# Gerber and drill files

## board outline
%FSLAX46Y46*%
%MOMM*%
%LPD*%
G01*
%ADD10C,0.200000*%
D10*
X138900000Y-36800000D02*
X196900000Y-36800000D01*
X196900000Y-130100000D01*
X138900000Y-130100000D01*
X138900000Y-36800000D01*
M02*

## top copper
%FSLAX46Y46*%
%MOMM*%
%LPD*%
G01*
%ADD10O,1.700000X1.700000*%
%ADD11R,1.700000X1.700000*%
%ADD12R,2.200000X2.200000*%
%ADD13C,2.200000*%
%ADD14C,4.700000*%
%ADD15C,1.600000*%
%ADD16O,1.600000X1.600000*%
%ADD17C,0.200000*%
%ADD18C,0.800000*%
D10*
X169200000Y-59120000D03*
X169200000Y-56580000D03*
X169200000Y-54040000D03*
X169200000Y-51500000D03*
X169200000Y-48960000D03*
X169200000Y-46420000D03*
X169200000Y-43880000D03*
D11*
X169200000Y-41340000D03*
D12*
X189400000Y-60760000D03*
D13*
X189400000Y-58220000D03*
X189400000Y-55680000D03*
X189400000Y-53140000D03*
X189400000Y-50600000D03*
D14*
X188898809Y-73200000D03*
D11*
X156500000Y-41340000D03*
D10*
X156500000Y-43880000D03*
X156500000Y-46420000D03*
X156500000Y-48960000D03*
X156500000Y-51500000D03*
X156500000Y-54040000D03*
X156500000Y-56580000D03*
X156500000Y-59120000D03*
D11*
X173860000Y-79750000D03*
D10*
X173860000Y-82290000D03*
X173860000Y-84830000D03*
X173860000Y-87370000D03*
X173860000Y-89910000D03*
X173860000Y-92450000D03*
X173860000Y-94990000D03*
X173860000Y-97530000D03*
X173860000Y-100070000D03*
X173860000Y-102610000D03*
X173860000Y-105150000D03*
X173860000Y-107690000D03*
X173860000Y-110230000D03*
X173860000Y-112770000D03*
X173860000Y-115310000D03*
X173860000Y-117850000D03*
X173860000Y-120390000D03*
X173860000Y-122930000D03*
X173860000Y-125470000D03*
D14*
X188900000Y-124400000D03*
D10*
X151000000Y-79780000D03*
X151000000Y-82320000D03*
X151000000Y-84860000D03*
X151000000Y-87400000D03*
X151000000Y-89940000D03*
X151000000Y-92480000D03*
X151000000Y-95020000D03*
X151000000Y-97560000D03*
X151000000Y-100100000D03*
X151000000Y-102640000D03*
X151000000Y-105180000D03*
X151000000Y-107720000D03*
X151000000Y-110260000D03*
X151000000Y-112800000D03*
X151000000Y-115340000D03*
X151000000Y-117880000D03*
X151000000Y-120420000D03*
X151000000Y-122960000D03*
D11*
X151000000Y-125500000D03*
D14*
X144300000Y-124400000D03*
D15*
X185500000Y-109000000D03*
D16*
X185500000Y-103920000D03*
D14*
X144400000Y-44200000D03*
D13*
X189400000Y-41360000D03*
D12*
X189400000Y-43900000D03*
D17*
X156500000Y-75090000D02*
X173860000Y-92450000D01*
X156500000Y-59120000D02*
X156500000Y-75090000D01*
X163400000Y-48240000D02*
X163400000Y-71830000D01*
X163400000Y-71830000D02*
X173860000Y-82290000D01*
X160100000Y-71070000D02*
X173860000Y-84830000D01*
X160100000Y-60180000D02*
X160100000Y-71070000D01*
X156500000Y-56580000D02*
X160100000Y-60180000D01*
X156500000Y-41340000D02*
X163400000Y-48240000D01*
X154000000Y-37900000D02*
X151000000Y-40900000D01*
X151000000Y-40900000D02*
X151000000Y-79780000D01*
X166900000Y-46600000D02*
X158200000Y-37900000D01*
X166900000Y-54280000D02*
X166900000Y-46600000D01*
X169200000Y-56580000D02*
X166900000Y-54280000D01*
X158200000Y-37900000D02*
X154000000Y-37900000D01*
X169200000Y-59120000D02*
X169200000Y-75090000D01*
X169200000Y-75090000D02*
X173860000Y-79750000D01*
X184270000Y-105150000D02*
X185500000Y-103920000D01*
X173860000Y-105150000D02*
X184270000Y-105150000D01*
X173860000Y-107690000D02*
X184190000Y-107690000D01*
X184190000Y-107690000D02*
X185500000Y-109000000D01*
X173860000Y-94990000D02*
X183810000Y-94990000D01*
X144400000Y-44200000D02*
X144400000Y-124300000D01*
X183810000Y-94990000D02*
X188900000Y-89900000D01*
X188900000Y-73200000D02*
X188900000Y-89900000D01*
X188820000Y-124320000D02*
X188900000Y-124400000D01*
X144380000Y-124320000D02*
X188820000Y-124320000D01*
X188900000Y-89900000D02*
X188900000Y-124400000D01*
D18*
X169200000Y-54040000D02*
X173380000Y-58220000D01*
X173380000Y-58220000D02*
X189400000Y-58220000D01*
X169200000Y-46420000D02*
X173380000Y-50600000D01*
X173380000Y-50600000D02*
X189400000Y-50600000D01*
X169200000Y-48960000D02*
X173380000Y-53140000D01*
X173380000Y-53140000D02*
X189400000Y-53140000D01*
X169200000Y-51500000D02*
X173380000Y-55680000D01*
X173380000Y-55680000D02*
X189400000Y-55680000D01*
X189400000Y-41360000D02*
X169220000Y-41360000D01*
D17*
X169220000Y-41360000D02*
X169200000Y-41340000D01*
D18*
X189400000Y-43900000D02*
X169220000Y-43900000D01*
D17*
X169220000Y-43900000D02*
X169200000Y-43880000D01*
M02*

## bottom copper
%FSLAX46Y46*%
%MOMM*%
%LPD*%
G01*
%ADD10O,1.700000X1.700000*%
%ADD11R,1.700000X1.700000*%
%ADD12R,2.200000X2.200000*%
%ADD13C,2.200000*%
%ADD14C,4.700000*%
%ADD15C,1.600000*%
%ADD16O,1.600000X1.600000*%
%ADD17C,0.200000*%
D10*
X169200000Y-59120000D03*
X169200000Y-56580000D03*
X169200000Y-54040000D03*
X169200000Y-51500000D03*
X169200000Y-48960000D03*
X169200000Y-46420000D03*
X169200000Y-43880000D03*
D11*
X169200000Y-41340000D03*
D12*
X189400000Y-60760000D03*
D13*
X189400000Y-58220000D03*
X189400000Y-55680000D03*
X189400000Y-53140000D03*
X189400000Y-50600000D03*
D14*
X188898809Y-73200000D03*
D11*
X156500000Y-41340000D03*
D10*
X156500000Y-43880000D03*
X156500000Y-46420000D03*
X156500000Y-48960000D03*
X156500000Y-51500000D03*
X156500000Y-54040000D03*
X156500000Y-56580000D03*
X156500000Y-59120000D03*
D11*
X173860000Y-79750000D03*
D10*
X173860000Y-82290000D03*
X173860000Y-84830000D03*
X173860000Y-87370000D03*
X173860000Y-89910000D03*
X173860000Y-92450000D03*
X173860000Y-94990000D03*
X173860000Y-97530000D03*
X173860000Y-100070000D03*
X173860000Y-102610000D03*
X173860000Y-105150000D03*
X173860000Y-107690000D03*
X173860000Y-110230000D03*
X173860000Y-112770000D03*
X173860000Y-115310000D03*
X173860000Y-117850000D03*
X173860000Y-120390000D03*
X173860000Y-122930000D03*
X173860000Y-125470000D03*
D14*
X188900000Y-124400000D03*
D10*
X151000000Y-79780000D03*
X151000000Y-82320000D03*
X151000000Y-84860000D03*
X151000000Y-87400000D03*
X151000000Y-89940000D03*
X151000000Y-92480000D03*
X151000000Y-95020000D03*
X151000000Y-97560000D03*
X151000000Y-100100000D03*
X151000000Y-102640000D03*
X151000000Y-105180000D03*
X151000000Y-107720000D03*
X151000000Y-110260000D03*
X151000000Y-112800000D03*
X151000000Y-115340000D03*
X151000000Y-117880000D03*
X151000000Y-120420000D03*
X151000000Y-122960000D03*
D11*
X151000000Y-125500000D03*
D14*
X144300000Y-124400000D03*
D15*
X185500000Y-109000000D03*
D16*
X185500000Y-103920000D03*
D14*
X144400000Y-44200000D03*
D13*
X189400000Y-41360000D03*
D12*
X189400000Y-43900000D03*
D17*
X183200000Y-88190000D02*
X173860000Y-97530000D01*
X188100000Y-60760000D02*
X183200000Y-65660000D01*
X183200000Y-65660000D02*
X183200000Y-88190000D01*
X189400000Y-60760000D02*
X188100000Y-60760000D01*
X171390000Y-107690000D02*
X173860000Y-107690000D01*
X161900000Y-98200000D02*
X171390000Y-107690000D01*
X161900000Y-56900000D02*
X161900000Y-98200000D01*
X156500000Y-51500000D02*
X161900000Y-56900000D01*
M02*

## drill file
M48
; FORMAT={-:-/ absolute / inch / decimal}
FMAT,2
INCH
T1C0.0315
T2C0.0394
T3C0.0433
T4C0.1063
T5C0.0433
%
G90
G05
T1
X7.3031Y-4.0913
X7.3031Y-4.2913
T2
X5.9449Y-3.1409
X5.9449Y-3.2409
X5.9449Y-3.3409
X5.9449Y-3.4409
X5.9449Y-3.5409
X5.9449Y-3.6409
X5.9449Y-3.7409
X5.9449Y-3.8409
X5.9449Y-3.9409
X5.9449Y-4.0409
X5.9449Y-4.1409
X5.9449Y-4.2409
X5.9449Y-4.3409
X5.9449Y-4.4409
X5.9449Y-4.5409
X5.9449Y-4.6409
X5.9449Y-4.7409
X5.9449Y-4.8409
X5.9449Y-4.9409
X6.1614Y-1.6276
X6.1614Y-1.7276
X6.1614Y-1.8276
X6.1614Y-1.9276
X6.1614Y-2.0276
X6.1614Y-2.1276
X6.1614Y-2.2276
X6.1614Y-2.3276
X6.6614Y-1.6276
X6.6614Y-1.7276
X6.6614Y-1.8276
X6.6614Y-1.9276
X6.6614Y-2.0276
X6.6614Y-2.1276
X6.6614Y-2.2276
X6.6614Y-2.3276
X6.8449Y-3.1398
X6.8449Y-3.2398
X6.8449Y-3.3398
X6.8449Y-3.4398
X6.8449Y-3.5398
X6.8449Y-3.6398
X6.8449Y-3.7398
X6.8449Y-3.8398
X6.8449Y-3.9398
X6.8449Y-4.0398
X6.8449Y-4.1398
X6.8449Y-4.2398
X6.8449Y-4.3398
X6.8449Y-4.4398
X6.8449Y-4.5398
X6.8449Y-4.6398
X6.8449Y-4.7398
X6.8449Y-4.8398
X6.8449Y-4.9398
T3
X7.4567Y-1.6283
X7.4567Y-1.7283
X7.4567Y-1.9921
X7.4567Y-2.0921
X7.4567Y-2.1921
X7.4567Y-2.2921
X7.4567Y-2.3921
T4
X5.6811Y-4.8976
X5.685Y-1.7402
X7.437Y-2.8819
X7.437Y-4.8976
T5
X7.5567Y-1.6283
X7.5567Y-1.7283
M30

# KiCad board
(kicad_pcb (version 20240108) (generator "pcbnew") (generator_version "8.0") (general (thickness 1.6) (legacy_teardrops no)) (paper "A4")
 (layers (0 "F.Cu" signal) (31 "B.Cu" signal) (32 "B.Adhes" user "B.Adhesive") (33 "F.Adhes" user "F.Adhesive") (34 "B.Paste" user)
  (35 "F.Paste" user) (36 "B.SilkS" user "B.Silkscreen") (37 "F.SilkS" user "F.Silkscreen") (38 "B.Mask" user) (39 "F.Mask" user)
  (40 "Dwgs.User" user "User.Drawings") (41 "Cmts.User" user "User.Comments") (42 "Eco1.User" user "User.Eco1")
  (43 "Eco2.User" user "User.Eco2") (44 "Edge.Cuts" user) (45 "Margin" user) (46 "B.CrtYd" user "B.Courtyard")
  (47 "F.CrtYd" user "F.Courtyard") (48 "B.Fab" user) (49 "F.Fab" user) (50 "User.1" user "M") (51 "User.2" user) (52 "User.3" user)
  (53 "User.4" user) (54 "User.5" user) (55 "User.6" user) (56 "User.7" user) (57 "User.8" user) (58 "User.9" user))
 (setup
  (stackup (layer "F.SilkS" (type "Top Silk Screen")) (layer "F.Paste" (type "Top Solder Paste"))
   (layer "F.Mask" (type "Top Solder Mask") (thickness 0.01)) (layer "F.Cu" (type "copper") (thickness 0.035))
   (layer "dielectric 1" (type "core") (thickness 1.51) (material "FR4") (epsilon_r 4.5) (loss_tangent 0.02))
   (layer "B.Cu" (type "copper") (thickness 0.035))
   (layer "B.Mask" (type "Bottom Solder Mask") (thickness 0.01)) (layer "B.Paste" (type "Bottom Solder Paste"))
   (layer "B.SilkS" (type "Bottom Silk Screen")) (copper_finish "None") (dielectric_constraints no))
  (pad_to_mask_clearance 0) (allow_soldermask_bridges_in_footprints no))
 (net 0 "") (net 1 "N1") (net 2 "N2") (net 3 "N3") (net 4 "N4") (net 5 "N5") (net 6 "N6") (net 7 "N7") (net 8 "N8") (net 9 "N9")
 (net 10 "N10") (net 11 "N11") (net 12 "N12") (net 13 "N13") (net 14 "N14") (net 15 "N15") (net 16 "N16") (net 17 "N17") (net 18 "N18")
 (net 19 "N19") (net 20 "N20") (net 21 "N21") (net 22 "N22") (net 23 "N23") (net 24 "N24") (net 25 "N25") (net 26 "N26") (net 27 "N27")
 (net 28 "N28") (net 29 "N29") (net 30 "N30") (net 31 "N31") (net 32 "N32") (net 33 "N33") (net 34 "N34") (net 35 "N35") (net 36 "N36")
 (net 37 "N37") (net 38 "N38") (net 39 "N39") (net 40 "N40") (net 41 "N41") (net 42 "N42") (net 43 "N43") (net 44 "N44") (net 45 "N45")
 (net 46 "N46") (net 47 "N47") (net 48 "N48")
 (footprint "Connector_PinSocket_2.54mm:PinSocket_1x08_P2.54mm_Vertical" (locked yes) (layer "F.Cu") (at 169.2 41.34)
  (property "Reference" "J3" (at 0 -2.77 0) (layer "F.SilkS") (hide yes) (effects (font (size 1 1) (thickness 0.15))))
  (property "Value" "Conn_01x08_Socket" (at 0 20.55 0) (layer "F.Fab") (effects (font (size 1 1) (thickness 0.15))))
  (pad "1" thru_hole rect (at 0 0) (size 1.7 1.7) (drill 1) (layers "*.Cu" "*.Mask") (remove_unused_layers no) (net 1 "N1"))
  (pad "2" thru_hole oval (at 0 2.54) (size 1.7 1.7) (drill 1) (layers "*.Cu" "*.Mask") (remove_unused_layers no) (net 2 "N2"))
  (pad "3" thru_hole oval (at 0 5.08) (size 1.7 1.7) (drill 1) (layers "*.Cu" "*.Mask") (remove_unused_layers no) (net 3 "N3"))
  (pad "4" thru_hole oval (at 0 7.62) (size 1.7 1.7) (drill 1) (layers "*.Cu" "*.Mask") (remove_unused_layers no) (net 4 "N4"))
  (pad "5" thru_hole oval (at 0 10.16) (size 1.7 1.7) (drill 1) (layers "*.Cu" "*.Mask") (remove_unused_layers no) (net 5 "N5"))
  (pad "6" thru_hole oval (at 0 12.7) (size 1.7 1.7) (drill 1) (layers "*.Cu" "*.Mask") (remove_unused_layers no) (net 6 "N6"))
  (pad "7" thru_hole oval (at 0 15.24) (size 1.7 1.7) (drill 1) (layers "*.Cu" "*.Mask") (remove_unused_layers no) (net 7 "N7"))
  (pad "8" thru_hole oval (at 0 17.78) (size 1.7 1.7) (drill 1) (layers "*.Cu" "*.Mask") (remove_unused_layers no) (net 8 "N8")))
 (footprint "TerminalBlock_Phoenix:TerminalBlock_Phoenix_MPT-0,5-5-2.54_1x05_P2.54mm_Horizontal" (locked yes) (layer "F.Cu")
  (at 189.4 60.76 90)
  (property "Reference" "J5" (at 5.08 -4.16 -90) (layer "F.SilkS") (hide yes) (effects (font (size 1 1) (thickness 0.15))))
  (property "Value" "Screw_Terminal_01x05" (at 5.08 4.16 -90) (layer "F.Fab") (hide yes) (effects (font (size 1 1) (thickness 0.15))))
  (pad "1" thru_hole rect (at 0 0 90) (size 2.2 2.2) (drill 1.1) (layers "*.Cu" "*.Mask") (remove_unused_layers no) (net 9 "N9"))
  (pad "2" thru_hole circle (at 2.54 0 90) (size 2.2 2.2) (drill 1.1) (layers "*.Cu" "*.Mask") (remove_unused_layers no) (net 6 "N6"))
  (pad "3" thru_hole circle (at 5.08 0 90) (size 2.2 2.2) (drill 1.1) (layers "*.Cu" "*.Mask") (remove_unused_layers no) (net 5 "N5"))
  (pad "4" thru_hole circle (at 7.62 0 90) (size 2.2 2.2) (drill 1.1) (layers "*.Cu" "*.Mask") (remove_unused_layers no) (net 4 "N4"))
  (pad "5" thru_hole circle (at 10.16 0 90) (size 2.2 2.2) (drill 1.1) (layers "*.Cu" "*.Mask") (remove_unused_layers no) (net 3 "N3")))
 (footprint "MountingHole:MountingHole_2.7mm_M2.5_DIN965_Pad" (layer "F.Cu") (at 188.898809 73.2)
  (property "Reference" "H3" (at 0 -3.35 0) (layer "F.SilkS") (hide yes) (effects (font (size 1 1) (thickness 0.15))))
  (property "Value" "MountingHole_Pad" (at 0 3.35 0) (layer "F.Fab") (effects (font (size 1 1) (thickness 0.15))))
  (pad "1" thru_hole circle (at 0 0) (size 4.7 4.7) (drill 2.7) (layers "*.Cu" "*.Mask") (remove_unused_layers no) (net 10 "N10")))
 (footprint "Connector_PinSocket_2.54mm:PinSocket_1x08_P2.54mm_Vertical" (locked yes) (layer "F.Cu") (at 156.5 41.34)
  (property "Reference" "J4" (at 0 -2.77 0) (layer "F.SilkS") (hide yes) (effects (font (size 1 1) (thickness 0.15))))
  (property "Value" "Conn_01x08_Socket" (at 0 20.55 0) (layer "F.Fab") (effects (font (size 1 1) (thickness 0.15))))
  (pad "1" thru_hole rect (at 0 0) (size 1.7 1.7) (drill 1) (layers "*.Cu" "*.Mask") (remove_unused_layers no) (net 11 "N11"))
  (pad "2" thru_hole oval (at 0 2.54) (size 1.7 1.7) (drill 1) (layers "*.Cu" "*.Mask") (remove_unused_layers no) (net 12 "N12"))
  (pad "3" thru_hole oval (at 0 5.08) (size 1.7 1.7) (drill 1) (layers "*.Cu" "*.Mask") (remove_unused_layers no) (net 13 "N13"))
  (pad "4" thru_hole oval (at 0 7.62) (size 1.7 1.7) (drill 1) (layers "*.Cu" "*.Mask") (remove_unused_layers no) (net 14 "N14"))
  (pad "5" thru_hole oval (at 0 10.16) (size 1.7 1.7) (drill 1) (layers "*.Cu" "*.Mask") (remove_unused_layers no) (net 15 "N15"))
  (pad "6" thru_hole oval (at 0 12.7) (size 1.7 1.7) (drill 1) (layers "*.Cu" "*.Mask") (remove_unused_layers no) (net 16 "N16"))
  (pad "7" thru_hole oval (at 0 15.24) (size 1.7 1.7) (drill 1) (layers "*.Cu" "*.Mask") (remove_unused_layers no) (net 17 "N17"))
  (pad "8" thru_hole oval (at 0 17.78) (size 1.7 1.7) (drill 1) (layers "*.Cu" "*.Mask") (remove_unused_layers no) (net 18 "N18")))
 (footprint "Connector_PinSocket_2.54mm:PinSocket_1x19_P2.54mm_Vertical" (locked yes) (layer "F.Cu") (at 173.86 79.75)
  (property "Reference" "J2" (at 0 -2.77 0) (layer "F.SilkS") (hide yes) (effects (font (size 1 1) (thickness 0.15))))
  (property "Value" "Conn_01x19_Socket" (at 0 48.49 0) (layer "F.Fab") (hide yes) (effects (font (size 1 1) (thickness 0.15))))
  (pad "1" thru_hole rect (at 0 0) (size 1.7 1.7) (drill 1) (layers "*.Cu" "*.Mask") (remove_unused_layers no) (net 8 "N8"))
  (pad "2" thru_hole oval (at 0 2.54) (size 1.7 1.7) (drill 1) (layers "*.Cu" "*.Mask") (remove_unused_layers no) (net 11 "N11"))
  (pad "3" thru_hole oval (at 0 5.08) (size 1.7 1.7) (drill 1) (layers "*.Cu" "*.Mask") (remove_unused_layers no) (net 17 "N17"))
  (pad "4" thru_hole oval (at 0 7.62) (size 1.7 1.7) (drill 1) (layers "*.Cu" "*.Mask") (remove_unused_layers no) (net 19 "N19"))
  (pad "5" thru_hole oval (at 0 10.16) (size 1.7 1.7) (drill 1) (layers "*.Cu" "*.Mask") (remove_unused_layers no) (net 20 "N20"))
  (pad "6" thru_hole oval (at 0 12.7) (size 1.7 1.7) (drill 1) (layers "*.Cu" "*.Mask") (remove_unused_layers no) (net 18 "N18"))
  (pad "7" thru_hole oval (at 0 15.24) (size 1.7 1.7) (drill 1) (layers "*.Cu" "*.Mask") (remove_unused_layers no) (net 10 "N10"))
  (pad "8" thru_hole oval (at 0 17.78) (size 1.7 1.7) (drill 1) (layers "*.Cu" "*.Mask") (remove_unused_layers no) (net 9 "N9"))
  (pad "9" thru_hole oval (at 0 20.32) (size 1.7 1.7) (drill 1) (layers "*.Cu" "*.Mask") (remove_unused_layers no) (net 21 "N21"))
  (pad "10" thru_hole oval (at 0 22.86) (size 1.7 1.7) (drill 1) (layers "*.Cu" "*.Mask") (remove_unused_layers no) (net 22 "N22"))
  (pad "11" thru_hole oval (at 0 25.4) (size 1.7 1.7) (drill 1) (layers "*.Cu" "*.Mask") (remove_unused_layers no) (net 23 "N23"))
  (pad "12" thru_hole oval (at 0 27.94) (size 1.7 1.7) (drill 1) (layers "*.Cu" "*.Mask") (remove_unused_layers no) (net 15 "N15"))
  (pad "13" thru_hole oval (at 0 30.48) (size 1.7 1.7) (drill 1) (layers "*.Cu" "*.Mask") (remove_unused_layers no) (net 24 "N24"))
  (pad "14" thru_hole oval (at 0 33.02) (size 1.7 1.7) (drill 1) (layers "*.Cu" "*.Mask") (remove_unused_layers no) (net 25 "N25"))
  (pad "15" thru_hole oval (at 0 35.56) (size 1.7 1.7) (drill 1) (layers "*.Cu" "*.Mask") (remove_unused_layers no) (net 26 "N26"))
  (pad "16" thru_hole oval (at 0 38.1) (size 1.7 1.7) (drill 1) (layers "*.Cu" "*.Mask") (remove_unused_layers no) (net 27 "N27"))
  (pad "17" thru_hole oval (at 0 40.64) (size 1.7 1.7) (drill 1) (layers "*.Cu" "*.Mask") (remove_unused_layers no) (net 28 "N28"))
  (pad "18" thru_hole oval (at 0 43.18) (size 1.7 1.7) (drill 1) (layers "*.Cu" "*.Mask") (remove_unused_layers no) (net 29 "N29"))
  (pad "19" thru_hole oval (at 0 45.72) (size 1.7 1.7) (drill 1) (layers "*.Cu" "*.Mask") (remove_unused_layers no) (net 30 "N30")))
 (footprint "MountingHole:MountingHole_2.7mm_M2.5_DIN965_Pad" (layer "F.Cu") (at 188.9 124.4)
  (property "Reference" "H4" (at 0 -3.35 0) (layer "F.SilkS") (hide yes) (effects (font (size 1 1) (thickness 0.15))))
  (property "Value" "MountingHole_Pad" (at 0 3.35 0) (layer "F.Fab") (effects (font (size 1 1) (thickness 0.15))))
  (pad "1" thru_hole circle (at 0 0) (size 4.7 4.7) (drill 2.7) (layers "*.Cu" "*.Mask") (remove_unused_layers no) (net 10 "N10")))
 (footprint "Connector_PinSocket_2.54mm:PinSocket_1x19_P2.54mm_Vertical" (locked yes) (layer "F.Cu") (at 151 125.5 180)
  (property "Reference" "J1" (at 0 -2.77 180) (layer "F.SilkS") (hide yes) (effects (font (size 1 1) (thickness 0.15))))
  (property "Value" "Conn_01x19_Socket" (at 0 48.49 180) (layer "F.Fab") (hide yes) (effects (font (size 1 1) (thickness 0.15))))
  (pad "1" thru_hole rect (at 0 0 180) (size 1.7 1.7) (drill 1) (layers "*.Cu" "*.Mask") (remove_unused_layers no) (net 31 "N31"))
  (pad "2" thru_hole oval (at 0 2.54 180) (size 1.7 1.7) (drill 1) (layers "*.Cu" "*.Mask") (remove_unused_layers no) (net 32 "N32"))
  (pad "3" thru_hole oval (at 0 5.08 180) (size 1.7 1.7) (drill 1) (layers "*.Cu" "*.Mask") (remove_unused_layers no) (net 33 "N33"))
  (pad "4" thru_hole oval (at 0 7.62 180) (size 1.7 1.7) (drill 1) (layers "*.Cu" "*.Mask") (remove_unused_layers no) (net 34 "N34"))
  (pad "5" thru_hole oval (at 0 10.16 180) (size 1.7 1.7) (drill 1) (layers "*.Cu" "*.Mask") (remove_unused_layers no) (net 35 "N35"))
  (pad "6" thru_hole oval (at 0 12.7 180) (size 1.7 1.7) (drill 1) (layers "*.Cu" "*.Mask") (remove_unused_layers no) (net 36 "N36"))
  (pad "7" thru_hole oval (at 0 15.24 180) (size 1.7 1.7) (drill 1) (layers "*.Cu" "*.Mask") (remove_unused_layers no) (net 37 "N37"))
  (pad "8" thru_hole oval (at 0 17.78 180) (size 1.7 1.7) (drill 1) (layers "*.Cu" "*.Mask") (remove_unused_layers no) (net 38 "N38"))
  (pad "9" thru_hole oval (at 0 20.32 180) (size 1.7 1.7) (drill 1) (layers "*.Cu" "*.Mask") (remove_unused_layers no) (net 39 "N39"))
  (pad "10" thru_hole oval (at 0 22.86 180) (size 1.7 1.7) (drill 1) (layers "*.Cu" "*.Mask") (remove_unused_layers no) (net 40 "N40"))
  (pad "11" thru_hole oval (at 0 25.4 180) (size 1.7 1.7) (drill 1) (layers "*.Cu" "*.Mask") (remove_unused_layers no) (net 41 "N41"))
  (pad "12" thru_hole oval (at 0 27.94 180) (size 1.7 1.7) (drill 1) (layers "*.Cu" "*.Mask") (remove_unused_layers no) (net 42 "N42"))
  (pad "13" thru_hole oval (at 0 30.48 180) (size 1.7 1.7) (drill 1) (layers "*.Cu" "*.Mask") (remove_unused_layers no) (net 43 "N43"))
  (pad "14" thru_hole oval (at 0 33.02 180) (size 1.7 1.7) (drill 1) (layers "*.Cu" "*.Mask") (remove_unused_layers no) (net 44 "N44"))
  (pad "15" thru_hole oval (at 0 35.56 180) (size 1.7 1.7) (drill 1) (layers "*.Cu" "*.Mask") (remove_unused_layers no) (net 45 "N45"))
  (pad "16" thru_hole oval (at 0 38.1 180) (size 1.7 1.7) (drill 1) (layers "*.Cu" "*.Mask") (remove_unused_layers no) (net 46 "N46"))
  (pad "17" thru_hole oval (at 0 40.64 180) (size 1.7 1.7) (drill 1) (layers "*.Cu" "*.Mask") (remove_unused_layers no) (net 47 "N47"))
  (pad "18" thru_hole oval (at 0 43.18 180) (size 1.7 1.7) (drill 1) (layers "*.Cu" "*.Mask") (remove_unused_layers no) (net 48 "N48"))
  (pad "19" thru_hole oval (at 0 45.72 180) (size 1.7 1.7) (drill 1) (layers "*.Cu" "*.Mask") (remove_unused_layers no) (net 7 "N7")))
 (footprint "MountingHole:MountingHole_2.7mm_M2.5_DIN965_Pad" (layer "F.Cu") (at 144.3 124.4)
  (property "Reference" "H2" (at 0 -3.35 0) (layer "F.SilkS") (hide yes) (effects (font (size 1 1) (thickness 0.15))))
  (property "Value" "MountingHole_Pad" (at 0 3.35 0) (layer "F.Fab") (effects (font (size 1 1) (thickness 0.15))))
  (pad "1" thru_hole circle (at 0 0) (size 4.7 4.7) (drill 2.7) (layers "*.Cu" "*.Mask") (remove_unused_layers no) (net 10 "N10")))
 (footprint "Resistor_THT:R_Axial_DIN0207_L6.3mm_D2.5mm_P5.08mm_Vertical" (layer "F.Cu") (at 185.5 109 90)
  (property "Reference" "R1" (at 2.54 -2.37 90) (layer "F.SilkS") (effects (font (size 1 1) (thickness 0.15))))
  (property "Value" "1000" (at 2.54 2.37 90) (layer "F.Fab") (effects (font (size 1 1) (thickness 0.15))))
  (pad "1" thru_hole circle (at 0 0 90) (size 1.6 1.6) (drill 0.8) (layers "*.Cu" "*.Mask") (remove_unused_layers no) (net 15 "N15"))
  (pad "2" thru_hole oval (at 5.08 0 90) (size 1.6 1.6) (drill 0.8) (layers "*.Cu" "*.Mask") (remove_unused_layers no) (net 23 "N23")))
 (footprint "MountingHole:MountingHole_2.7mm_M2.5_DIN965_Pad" (layer "F.Cu") (at 144.4 44.2)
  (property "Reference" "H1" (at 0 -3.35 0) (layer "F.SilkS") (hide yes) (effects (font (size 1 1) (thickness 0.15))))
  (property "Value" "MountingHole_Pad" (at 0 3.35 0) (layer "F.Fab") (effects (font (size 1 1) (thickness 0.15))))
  (pad "1" thru_hole circle (at 0 0) (size 4.7 4.7) (drill 2.7) (layers "*.Cu" "*.Mask") (remove_unused_layers no) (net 10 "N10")))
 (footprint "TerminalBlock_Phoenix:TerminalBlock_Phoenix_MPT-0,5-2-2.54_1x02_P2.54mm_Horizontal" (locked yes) (layer "F.Cu")
  (at 189.4 43.9 90)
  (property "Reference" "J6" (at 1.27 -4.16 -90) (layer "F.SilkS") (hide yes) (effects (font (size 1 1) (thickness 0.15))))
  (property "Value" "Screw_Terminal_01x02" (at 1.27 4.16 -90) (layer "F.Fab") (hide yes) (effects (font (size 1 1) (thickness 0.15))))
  (pad "" np_thru_hole circle (at 0 2.54 90) (size 1.1 1.1) (drill 1.1) (layers "*.Cu" "*.Mask"))
  (pad "" np_thru_hole circle (at 2.54 2.54 90) (size 1.1 1.1) (drill 1.1) (layers "*.Cu" "*.Mask"))
  (pad "1" thru_hole rect (at 0 0 90) (size 2.2 2.2) (drill 1.1) (layers "*.Cu" "*.Mask") (remove_unused_layers no) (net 2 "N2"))
  (pad "2" thru_hole circle (at 2.54 0 90) (size 2.2 2.2) (drill 1.1) (layers "*.Cu" "*.Mask") (remove_unused_layers no) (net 1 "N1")))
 (gr_rect (start 138.9 36.8) (end 196.9 130.1) (stroke (width 0.2) (type default)) (fill none) (layer "Edge.Cuts"))
 (segment (start 151 40.9) (end 151 79.78) (width 0.2) (layer "F.Cu") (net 7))
 (segment (start 158.2 37.9) (end 154 37.9) (width 0.2) (layer "F.Cu") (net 7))
 (segment (start 154 37.9) (end 151 40.9) (width 0.2) (layer "F.Cu") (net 7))
 (segment (start 166.9 54.28) (end 166.9 46.6) (width 0.2) (layer "F.Cu") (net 7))
 (segment (start 166.9 46.6) (end 158.2 37.9) (width 0.2) (layer "F.Cu") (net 7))
 (segment (start 169.2 56.58) (end 166.9 54.28) (width 0.2) (layer "F.Cu") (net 7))
 (segment (start 169.2 59.12) (end 169.2 75.09) (width 0.2) (layer "F.Cu") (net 8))
 (segment (start 169.2 75.09) (end 173.86 79.75) (width 0.2) (layer "F.Cu") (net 8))
 (segment (start 183.2 65.66) (end 183.2 88.19) (width 0.2) (layer "B.Cu") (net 9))
 (segment (start 183.2 88.19) (end 173.86 97.53) (width 0.2) (layer "B.Cu") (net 9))
 (segment (start 188.1 60.76) (end 183.2 65.66) (width 0.2) (layer "B.Cu") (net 9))
 (segment (start 189.4 60.76) (end 188.1 60.76) (width 0.2) (layer "B.Cu") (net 9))
 (segment (start 160.1 60.18) (end 160.1 71.07) (width 0.2) (layer "F.Cu") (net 17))
 (segment (start 156.5 56.58) (end 160.1 60.18) (width 0.2) (layer "F.Cu") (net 17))
 (segment (start 160.1 71.07) (end 173.86 84.83) (width 0.2) (layer "F.Cu") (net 17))
 (segment (start 156.5 75.09) (end 173.86 92.45) (width 0.2) (layer "F.Cu") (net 18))
 (segment (start 156.5 59.12) (end 156.5 75.09) (width 0.2) (layer "F.Cu") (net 18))
 (segment (start 163.4 48.24) (end 163.4 71.83) (width 0.2) (layer "F.Cu") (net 11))
 (segment (start 156.5 41.34) (end 163.4 48.24) (width 0.2) (layer "F.Cu") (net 11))
 (segment (start 163.4 71.83) (end 173.86 82.29) (width 0.2) (layer "F.Cu") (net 11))
 (segment (start 184.27 105.15) (end 185.5 103.92) (width 0.2) (layer "F.Cu") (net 23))
 (segment (start 173.86 105.15) (end 184.27 105.15) (width 0.2) (layer "F.Cu") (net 23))
 (segment (start 173.86 107.69) (end 184.19 107.69) (width 0.2) (layer "F.Cu") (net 15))
 (segment (start 184.19 107.69) (end 185.5 109) (width 0.2) (layer "F.Cu") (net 15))
 (segment (start 161.9 98.2) (end 171.39 107.69) (width 0.2) (layer "B.Cu") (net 15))
 (segment (start 161.9 56.9) (end 161.9 98.2) (width 0.2) (layer "B.Cu") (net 15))
 (segment (start 156.5 51.5) (end 161.9 56.9) (width 0.2) (layer "B.Cu") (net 15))
 (segment (start 171.39 107.69) (end 173.86 107.69) (width 0.2) (layer "B.Cu") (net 15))
 (segment (start 173.86 94.99) (end 183.81 94.99) (width 0.2) (layer "F.Cu") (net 10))
 (segment (start 144.4 44.2) (end 144.4 124.3) (width 0.2) (layer "F.Cu") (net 10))
 (segment (start 183.81 94.99) (end 188.9 89.9) (width 0.2) (layer "F.Cu") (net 10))
 (segment (start 188.9 73.2) (end 188.9 89.9) (width 0.2) (layer "F.Cu") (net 10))
 (segment (start 188.82 124.32) (end 188.9 124.4) (width 0.2) (layer "F.Cu") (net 10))
 (segment (start 144.38 124.32) (end 188.82 124.32) (width 0.2) (layer "F.Cu") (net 10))
 (segment (start 188.9 89.9) (end 188.9 124.4) (width 0.2) (layer "F.Cu") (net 10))
 (segment (start 169.2 54.04) (end 173.38 58.22) (width 0.8) (layer "F.Cu") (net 6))
 (segment (start 173.38 58.22) (end 189.4 58.22) (width 0.8) (layer "F.Cu") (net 6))
 (segment (start 169.2 46.42) (end 173.38 50.6) (width 0.8) (layer "F.Cu") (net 3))
 (segment (start 173.38 50.6) (end 189.4 50.6) (width 0.8) (layer "F.Cu") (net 3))
 (segment (start 169.2 48.96) (end 173.38 53.14) (width 0.8) (layer "F.Cu") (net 4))
 (segment (start 173.38 53.14) (end 189.4 53.14) (width 0.8) (layer "F.Cu") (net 4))
 (segment (start 169.2 51.5) (end 173.38 55.68) (width 0.8) (layer "F.Cu") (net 5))
 (segment (start 173.38 55.68) (end 189.4 55.68) (width 0.8) (layer "F.Cu") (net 5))
 (segment (start 189.4 41.36) (end 169.22 41.36) (width 0.8) (layer "F.Cu") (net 1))
 (segment (start 169.22 41.36) (end 169.2 41.34) (width 0.2) (layer "F.Cu") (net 1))
 (segment (start 189.4 43.9) (end 169.22 43.9) (width 0.8) (layer "F.Cu") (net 2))
 (segment (start 169.22 43.9) (end 169.2 43.88) (width 0.2) (layer "F.Cu") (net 2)))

